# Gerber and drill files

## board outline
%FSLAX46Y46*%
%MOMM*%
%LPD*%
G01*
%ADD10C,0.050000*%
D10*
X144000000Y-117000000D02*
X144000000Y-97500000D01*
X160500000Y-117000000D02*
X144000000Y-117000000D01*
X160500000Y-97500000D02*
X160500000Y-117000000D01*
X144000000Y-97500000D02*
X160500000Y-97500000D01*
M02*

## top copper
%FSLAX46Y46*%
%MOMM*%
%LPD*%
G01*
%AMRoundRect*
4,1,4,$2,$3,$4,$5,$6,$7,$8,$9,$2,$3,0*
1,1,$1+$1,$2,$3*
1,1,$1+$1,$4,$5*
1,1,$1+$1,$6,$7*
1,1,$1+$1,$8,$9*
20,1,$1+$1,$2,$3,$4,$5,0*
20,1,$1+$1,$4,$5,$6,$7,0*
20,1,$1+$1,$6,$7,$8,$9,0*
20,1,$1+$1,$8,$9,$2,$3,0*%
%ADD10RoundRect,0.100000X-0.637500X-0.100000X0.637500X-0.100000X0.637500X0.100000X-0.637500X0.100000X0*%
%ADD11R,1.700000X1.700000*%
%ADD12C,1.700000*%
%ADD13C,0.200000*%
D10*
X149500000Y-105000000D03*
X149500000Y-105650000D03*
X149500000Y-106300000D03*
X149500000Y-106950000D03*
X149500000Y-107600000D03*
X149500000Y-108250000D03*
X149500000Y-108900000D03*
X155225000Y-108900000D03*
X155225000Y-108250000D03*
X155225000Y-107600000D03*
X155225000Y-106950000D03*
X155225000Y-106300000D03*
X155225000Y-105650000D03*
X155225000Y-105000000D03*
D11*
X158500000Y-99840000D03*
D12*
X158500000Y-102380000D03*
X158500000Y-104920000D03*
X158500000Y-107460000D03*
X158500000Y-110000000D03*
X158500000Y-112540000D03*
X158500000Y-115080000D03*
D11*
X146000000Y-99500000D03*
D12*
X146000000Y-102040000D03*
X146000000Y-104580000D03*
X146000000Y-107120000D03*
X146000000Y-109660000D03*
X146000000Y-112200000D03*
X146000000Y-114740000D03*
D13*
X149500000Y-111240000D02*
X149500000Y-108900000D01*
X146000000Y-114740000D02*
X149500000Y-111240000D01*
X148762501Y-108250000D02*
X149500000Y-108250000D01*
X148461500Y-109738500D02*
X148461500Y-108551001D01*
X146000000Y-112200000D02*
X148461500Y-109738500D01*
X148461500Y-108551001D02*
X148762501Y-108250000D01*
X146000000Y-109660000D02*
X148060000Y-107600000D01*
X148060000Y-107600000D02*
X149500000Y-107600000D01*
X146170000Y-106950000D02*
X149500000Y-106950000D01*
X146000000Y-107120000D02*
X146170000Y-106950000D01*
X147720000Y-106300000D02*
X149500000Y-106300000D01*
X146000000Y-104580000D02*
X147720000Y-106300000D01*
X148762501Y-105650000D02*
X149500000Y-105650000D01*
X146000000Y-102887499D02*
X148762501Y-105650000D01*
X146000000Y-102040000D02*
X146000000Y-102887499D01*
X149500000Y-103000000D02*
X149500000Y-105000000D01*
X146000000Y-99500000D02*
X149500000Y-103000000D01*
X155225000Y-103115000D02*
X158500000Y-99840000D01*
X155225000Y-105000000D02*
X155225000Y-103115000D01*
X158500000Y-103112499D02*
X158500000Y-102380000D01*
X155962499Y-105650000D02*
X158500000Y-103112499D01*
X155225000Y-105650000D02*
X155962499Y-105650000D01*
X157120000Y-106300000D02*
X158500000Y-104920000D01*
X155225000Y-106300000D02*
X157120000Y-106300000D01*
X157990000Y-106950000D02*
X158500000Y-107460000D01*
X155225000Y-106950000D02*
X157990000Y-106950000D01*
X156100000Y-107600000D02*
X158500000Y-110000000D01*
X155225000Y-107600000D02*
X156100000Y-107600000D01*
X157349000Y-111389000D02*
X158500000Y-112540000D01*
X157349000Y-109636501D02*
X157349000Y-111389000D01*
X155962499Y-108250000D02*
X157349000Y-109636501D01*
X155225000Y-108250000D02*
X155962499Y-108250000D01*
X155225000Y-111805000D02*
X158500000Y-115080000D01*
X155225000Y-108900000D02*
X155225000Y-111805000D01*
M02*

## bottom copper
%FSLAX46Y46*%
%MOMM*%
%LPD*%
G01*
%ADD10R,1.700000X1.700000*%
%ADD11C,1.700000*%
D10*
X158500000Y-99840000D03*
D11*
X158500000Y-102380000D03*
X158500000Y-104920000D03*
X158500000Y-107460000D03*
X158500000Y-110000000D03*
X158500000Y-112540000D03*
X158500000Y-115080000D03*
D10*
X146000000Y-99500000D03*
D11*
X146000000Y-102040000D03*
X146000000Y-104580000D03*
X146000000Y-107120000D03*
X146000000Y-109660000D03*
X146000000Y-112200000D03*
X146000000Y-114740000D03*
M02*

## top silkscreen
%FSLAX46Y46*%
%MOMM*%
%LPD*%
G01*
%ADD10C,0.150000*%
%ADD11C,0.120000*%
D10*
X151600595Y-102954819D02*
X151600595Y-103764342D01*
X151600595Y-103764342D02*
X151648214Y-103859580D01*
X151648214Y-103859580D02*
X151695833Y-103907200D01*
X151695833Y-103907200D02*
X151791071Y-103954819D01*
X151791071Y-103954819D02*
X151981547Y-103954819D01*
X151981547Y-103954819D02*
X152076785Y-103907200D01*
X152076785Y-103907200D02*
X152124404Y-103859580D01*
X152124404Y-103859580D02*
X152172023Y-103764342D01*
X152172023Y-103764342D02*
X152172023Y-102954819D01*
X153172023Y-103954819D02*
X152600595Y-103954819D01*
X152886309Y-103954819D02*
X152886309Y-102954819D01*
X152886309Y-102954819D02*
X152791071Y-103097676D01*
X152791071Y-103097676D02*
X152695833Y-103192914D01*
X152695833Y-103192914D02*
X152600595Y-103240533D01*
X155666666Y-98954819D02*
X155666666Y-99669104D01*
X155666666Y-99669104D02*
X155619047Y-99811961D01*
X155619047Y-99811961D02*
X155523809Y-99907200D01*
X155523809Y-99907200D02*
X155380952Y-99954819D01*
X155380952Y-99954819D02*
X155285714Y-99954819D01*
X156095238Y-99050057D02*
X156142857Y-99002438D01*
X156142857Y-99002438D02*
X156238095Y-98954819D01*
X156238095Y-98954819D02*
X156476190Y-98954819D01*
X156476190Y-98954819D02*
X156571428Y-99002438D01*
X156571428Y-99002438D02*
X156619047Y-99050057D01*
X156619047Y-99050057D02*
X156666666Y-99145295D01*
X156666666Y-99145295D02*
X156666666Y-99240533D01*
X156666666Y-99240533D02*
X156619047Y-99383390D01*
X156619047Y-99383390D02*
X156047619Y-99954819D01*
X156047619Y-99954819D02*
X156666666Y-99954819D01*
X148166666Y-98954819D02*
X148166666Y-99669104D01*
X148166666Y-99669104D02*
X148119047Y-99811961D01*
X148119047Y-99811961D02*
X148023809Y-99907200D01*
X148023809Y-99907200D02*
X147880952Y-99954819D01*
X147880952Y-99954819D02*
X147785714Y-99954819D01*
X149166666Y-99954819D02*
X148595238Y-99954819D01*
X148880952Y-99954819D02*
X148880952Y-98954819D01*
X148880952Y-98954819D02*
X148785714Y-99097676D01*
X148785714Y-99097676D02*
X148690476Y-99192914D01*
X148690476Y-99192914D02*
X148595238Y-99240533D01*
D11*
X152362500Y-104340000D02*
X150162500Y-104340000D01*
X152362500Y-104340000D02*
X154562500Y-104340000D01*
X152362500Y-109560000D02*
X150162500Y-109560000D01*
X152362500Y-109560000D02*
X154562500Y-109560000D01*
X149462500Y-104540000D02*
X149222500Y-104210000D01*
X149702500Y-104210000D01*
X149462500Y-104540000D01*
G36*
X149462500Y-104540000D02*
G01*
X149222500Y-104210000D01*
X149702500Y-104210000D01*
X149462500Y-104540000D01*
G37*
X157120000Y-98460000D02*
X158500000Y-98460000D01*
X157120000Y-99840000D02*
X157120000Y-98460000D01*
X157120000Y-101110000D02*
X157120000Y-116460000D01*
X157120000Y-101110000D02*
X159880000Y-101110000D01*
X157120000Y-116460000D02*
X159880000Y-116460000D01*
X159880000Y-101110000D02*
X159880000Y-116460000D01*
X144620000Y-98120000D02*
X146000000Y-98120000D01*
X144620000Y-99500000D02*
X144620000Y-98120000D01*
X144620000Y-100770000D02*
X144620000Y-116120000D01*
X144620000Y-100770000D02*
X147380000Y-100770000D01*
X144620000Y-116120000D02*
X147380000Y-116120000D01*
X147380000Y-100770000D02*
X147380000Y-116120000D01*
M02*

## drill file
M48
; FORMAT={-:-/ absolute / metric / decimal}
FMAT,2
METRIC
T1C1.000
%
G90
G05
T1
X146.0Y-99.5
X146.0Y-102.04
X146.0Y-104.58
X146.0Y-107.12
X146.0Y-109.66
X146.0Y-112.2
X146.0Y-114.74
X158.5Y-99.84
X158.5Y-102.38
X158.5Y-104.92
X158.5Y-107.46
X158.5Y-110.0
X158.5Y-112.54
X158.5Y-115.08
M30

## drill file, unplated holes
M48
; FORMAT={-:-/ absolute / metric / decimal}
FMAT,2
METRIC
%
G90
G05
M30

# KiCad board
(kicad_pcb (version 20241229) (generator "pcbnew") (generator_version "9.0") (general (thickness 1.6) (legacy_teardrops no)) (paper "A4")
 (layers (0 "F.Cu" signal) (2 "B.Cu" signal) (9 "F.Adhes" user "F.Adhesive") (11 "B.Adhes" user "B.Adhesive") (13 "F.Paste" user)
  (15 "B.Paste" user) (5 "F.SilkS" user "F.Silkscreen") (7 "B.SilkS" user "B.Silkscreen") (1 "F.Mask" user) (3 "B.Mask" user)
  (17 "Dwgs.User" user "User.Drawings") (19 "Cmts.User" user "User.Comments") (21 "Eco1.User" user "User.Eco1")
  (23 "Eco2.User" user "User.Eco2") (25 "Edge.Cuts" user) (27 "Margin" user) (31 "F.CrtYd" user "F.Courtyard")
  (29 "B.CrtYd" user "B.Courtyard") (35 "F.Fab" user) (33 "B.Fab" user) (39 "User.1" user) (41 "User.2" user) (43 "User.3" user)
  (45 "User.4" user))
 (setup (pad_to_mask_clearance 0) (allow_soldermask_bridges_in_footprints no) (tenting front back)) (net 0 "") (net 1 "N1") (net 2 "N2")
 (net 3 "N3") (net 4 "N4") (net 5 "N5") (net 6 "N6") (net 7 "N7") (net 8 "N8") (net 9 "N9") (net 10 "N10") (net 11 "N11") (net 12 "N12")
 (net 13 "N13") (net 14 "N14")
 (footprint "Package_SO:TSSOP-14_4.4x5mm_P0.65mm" (layer "F.Cu") (at 152.3625 106.95)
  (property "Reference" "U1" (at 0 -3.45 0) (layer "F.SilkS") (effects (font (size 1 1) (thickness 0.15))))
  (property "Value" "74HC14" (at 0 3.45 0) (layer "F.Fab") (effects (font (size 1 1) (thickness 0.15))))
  (fp_line (start 0 -2.61) (end -2.2 -2.61) (stroke (width 0.12) (type solid)) (layer "F.SilkS"))
  (fp_line (start 0 -2.61) (end 2.2 -2.61) (stroke (width 0.12) (type solid)) (layer "F.SilkS"))
  (fp_line (start 0 2.61) (end -2.2 2.61) (stroke (width 0.12) (type solid)) (layer "F.SilkS"))
  (fp_line (start 0 2.61) (end 2.2 2.61) (stroke (width 0.12) (type solid)) (layer "F.SilkS"))
  (fp_poly (pts (xy -2.9 -2.41) (xy -3.14 -2.74) (xy -2.66 -2.74)) (stroke (width 0.12) (type solid)) (fill yes) (layer "F.SilkS"))
  (pad "1" smd roundrect (at -2.8625 -1.95) (size 1.475 0.4) (layers "F.Cu" "F.Mask" "F.Paste") (roundrect_rratio 0.25) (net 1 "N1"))
  (pad "2" smd roundrect (at -2.8625 -1.3) (size 1.475 0.4) (layers "F.Cu" "F.Mask" "F.Paste") (roundrect_rratio 0.25) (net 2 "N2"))
  (pad "3" smd roundrect (at -2.8625 -0.65) (size 1.475 0.4) (layers "F.Cu" "F.Mask" "F.Paste") (roundrect_rratio 0.25) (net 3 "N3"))
  (pad "4" smd roundrect (at -2.8625 0) (size 1.475 0.4) (layers "F.Cu" "F.Mask" "F.Paste") (roundrect_rratio 0.25) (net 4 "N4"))
  (pad "5" smd roundrect (at -2.8625 0.65) (size 1.475 0.4) (layers "F.Cu" "F.Mask" "F.Paste") (roundrect_rratio 0.25) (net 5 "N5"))
  (pad "6" smd roundrect (at -2.8625 1.3) (size 1.475 0.4) (layers "F.Cu" "F.Mask" "F.Paste") (roundrect_rratio 0.25) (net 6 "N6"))
  (pad "7" smd roundrect (at -2.8625 1.95) (size 1.475 0.4) (layers "F.Cu" "F.Mask" "F.Paste") (roundrect_rratio 0.25) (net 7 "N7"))
  (pad "8" smd roundrect (at 2.8625 1.95) (size 1.475 0.4) (layers "F.Cu" "F.Mask" "F.Paste") (roundrect_rratio 0.25) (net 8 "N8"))
  (pad "9" smd roundrect (at 2.8625 1.3) (size 1.475 0.4) (layers "F.Cu" "F.Mask" "F.Paste") (roundrect_rratio 0.25) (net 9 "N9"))
  (pad "10" smd roundrect (at 2.8625 0.65) (size 1.475 0.4) (layers "F.Cu" "F.Mask" "F.Paste") (roundrect_rratio 0.25) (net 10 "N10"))
  (pad "11" smd roundrect (at 2.8625 0) (size 1.475 0.4) (layers "F.Cu" "F.Mask" "F.Paste") (roundrect_rratio 0.25) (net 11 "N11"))
  (pad "12" smd roundrect (at 2.8625 -0.65) (size 1.475 0.4) (layers "F.Cu" "F.Mask" "F.Paste") (roundrect_rratio 0.25) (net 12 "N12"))
  (pad "13" smd roundrect (at 2.8625 -1.3) (size 1.475 0.4) (layers "F.Cu" "F.Mask" "F.Paste") (roundrect_rratio 0.25) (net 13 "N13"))
  (pad "14" smd roundrect (at 2.8625 -1.95) (size 1.475 0.4) (layers "F.Cu" "F.Mask" "F.Paste") (roundrect_rratio 0.25) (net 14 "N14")))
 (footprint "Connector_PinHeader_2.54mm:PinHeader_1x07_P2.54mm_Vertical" (layer "F.Cu") (at 146 99.5)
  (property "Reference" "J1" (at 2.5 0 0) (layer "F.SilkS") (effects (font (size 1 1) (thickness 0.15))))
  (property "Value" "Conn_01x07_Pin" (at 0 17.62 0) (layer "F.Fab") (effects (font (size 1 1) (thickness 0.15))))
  (fp_line (start -1.38 -1.38) (end 0 -1.38) (stroke (width 0.12) (type solid)) (layer "F.SilkS"))
  (fp_line (start -1.38 0) (end -1.38 -1.38) (stroke (width 0.12) (type solid)) (layer "F.SilkS"))
  (fp_line (start -1.38 1.27) (end -1.38 16.62) (stroke (width 0.12) (type solid)) (layer "F.SilkS"))
  (fp_line (start -1.38 1.27) (end 1.38 1.27) (stroke (width 0.12) (type solid)) (layer "F.SilkS"))
  (fp_line (start -1.38 16.62) (end 1.38 16.62) (stroke (width 0.12) (type solid)) (layer "F.SilkS"))
  (fp_line (start 1.38 1.27) (end 1.38 16.62) (stroke (width 0.12) (type solid)) (layer "F.SilkS"))
  (pad "1" thru_hole rect (at 0 0) (size 1.7 1.7) (drill 1) (layers "*.Cu" "*.Mask") (remove_unused_layers no) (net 1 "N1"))
  (pad "2" thru_hole circle (at 0 2.54) (size 1.7 1.7) (drill 1) (layers "*.Cu" "*.Mask") (remove_unused_layers no) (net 2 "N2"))
  (pad "3" thru_hole circle (at 0 5.08) (size 1.7 1.7) (drill 1) (layers "*.Cu" "*.Mask") (remove_unused_layers no) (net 3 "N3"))
  (pad "4" thru_hole circle (at 0 7.62) (size 1.7 1.7) (drill 1) (layers "*.Cu" "*.Mask") (remove_unused_layers no) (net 4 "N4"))
  (pad "5" thru_hole circle (at 0 10.16) (size 1.7 1.7) (drill 1) (layers "*.Cu" "*.Mask") (remove_unused_layers no) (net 5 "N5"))
  (pad "6" thru_hole circle (at 0 12.7) (size 1.7 1.7) (drill 1) (layers "*.Cu" "*.Mask") (remove_unused_layers no) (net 6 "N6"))
  (pad "7" thru_hole circle (at 0 15.24) (size 1.7 1.7) (drill 1) (layers "*.Cu" "*.Mask") (remove_unused_layers no) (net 7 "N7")))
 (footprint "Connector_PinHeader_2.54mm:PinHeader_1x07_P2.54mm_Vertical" (layer "F.Cu") (at 158.5 99.84)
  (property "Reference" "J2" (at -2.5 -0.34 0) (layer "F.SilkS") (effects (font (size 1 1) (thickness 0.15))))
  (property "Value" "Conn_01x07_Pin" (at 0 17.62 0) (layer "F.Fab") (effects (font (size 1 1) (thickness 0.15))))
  (fp_line (start -1.38 -1.38) (end 0 -1.38) (stroke (width 0.12) (type solid)) (layer "F.SilkS"))
  (fp_line (start -1.38 0) (end -1.38 -1.38) (stroke (width 0.12) (type solid)) (layer "F.SilkS"))
  (fp_line (start -1.38 1.27) (end -1.38 16.62) (stroke (width 0.12) (type solid)) (layer "F.SilkS"))
  (fp_line (start -1.38 1.27) (end 1.38 1.27) (stroke (width 0.12) (type solid)) (layer "F.SilkS"))
  (fp_line (start -1.38 16.62) (end 1.38 16.62) (stroke (width 0.12) (type solid)) (layer "F.SilkS"))
  (fp_line (start 1.38 1.27) (end 1.38 16.62) (stroke (width 0.12) (type solid)) (layer "F.SilkS"))
  (pad "1" thru_hole rect (at 0 0) (size 1.7 1.7) (drill 1) (layers "*.Cu" "*.Mask") (remove_unused_layers no) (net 14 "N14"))
  (pad "2" thru_hole circle (at 0 2.54) (size 1.7 1.7) (drill 1) (layers "*.Cu" "*.Mask") (remove_unused_layers no) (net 13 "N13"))
  (pad "3" thru_hole circle (at 0 5.08) (size 1.7 1.7) (drill 1) (layers "*.Cu" "*.Mask") (remove_unused_layers no) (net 12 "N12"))
  (pad "4" thru_hole circle (at 0 7.62) (size 1.7 1.7) (drill 1) (layers "*.Cu" "*.Mask") (remove_unused_layers no) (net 11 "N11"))
  (pad "5" thru_hole circle (at 0 10.16) (size 1.7 1.7) (drill 1) (layers "*.Cu" "*.Mask") (remove_unused_layers no) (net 10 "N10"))
  (pad "6" thru_hole circle (at 0 12.7) (size 1.7 1.7) (drill 1) (layers "*.Cu" "*.Mask") (remove_unused_layers no) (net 9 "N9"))
  (pad "7" thru_hole circle (at 0 15.24) (size 1.7 1.7) (drill 1) (layers "*.Cu" "*.Mask") (remove_unused_layers no) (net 8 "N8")))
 (gr_line (start 144 117) (end 144 97.5) (stroke (width 0.05) (type default)) (layer "Edge.Cuts"))
 (gr_line (start 160.5 97.5) (end 160.5 117) (stroke (width 0.05) (type default)) (layer "Edge.Cuts"))
 (gr_line (start 160.5 117) (end 144 117) (stroke (width 0.05) (type default)) (layer "Edge.Cuts"))
 (gr_line (start 144 97.5) (end 160.5 97.5) (stroke (width 0.05) (type default)) (layer "Edge.Cuts"))
 (segment (start 148.06 107.6) (end 149.5 107.6) (width 0.2) (layer "F.Cu") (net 5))
 (segment (start 146 109.66) (end 148.06 107.6) (width 0.2) (layer "F.Cu") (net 5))
 (segment (start 149.5 103) (end 149.5 105) (width 0.2) (layer "F.Cu") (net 1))
 (segment (start 146 99.5) (end 149.5 103) (width 0.2) (layer "F.Cu") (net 1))
 (segment (start 146 112.2) (end 148.4615 109.7385) (width 0.2) (layer "F.Cu") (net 6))
 (segment (start 148.4615 109.7385) (end 148.4615 108.551001) (width 0.2) (layer "F.Cu") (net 6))
 (segment (start 148.4615 108.551001) (end 148.762501 108.25) (width 0.2) (layer "F.Cu") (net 6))
 (segment (start 148.762501 108.25) (end 149.5 108.25) (width 0.2) (layer "F.Cu") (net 6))
 (segment (start 146 104.58) (end 147.72 106.3) (width 0.2) (layer "F.Cu") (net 3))
 (segment (start 147.72 106.3) (end 149.5 106.3) (width 0.2) (layer "F.Cu") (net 3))
 (segment (start 146 102.04) (end 146 102.887499) (width 0.2) (layer "F.Cu") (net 2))
 (segment (start 148.762501 105.65) (end 149.5 105.65) (width 0.2) (layer "F.Cu") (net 2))
 (segment (start 146 102.887499) (end 148.762501 105.65) (width 0.2) (layer "F.Cu") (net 2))
 (segment (start 146 107.12) (end 146.17 106.95) (width 0.2) (layer "F.Cu") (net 4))
 (segment (start 146.17 106.95) (end 149.5 106.95) (width 0.2) (layer "F.Cu") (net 4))
 (segment (start 146 114.74) (end 149.5 111.24) (width 0.2) (layer "F.Cu") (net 7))
 (segment (start 149.5 111.24) (end 149.5 108.9) (width 0.2) (layer "F.Cu") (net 7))
 (segment (start 155.962499 105.65) (end 158.5 103.112499) (width 0.2) (layer "F.Cu") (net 13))
 (segment (start 158.5 103.112499) (end 158.5 102.38) (width 0.2) (layer "F.Cu") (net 13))
 (segment (start 155.225 105.65) (end 155.962499 105.65) (width 0.2) (layer "F.Cu") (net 13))
 (segment (start 155.225 106.3) (end 157.12 106.3) (width 0.2) (layer "F.Cu") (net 12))
 (segment (start 157.12 106.3) (end 158.5 104.92) (width 0.2) (layer "F.Cu") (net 12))
 (segment (start 155.225 111.805) (end 158.5 115.08) (width 0.2) (layer "F.Cu") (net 8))
 (segment (start 155.225 108.9) (end 155.225 111.805) (width 0.2) (layer "F.Cu") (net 8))
 (segment (start 155.225 105) (end 155.225 103.115) (width 0.2) (layer "F.Cu") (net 14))
 (segment (start 155.225 103.115) (end 158.5 99.84) (width 0.2) (layer "F.Cu") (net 14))
 (segment (start 157.99 106.95) (end 158.5 107.46) (width 0.2) (layer "F.Cu") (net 11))
 (segment (start 155.225 106.95) (end 157.99 106.95) (width 0.2) (layer "F.Cu") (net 11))
 (segment (start 157.349 111.389) (end 158.5 112.54) (width 0.2) (layer "F.Cu") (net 9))
 (segment (start 157.349 109.636501) (end 157.349 111.389) (width 0.2) (layer "F.Cu") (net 9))
 (segment (start 155.225 108.25) (end 155.962499 108.25) (width 0.2) (layer "F.Cu") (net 9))
 (segment (start 155.962499 108.25) (end 157.349 109.636501) (width 0.2) (layer "F.Cu") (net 9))
 (segment (start 156.1 107.6) (end 158.5 110) (width 0.2) (layer "F.Cu") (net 10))
 (segment (start 155.225 107.6) (end 156.1 107.6) (width 0.2) (layer "F.Cu") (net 10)))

